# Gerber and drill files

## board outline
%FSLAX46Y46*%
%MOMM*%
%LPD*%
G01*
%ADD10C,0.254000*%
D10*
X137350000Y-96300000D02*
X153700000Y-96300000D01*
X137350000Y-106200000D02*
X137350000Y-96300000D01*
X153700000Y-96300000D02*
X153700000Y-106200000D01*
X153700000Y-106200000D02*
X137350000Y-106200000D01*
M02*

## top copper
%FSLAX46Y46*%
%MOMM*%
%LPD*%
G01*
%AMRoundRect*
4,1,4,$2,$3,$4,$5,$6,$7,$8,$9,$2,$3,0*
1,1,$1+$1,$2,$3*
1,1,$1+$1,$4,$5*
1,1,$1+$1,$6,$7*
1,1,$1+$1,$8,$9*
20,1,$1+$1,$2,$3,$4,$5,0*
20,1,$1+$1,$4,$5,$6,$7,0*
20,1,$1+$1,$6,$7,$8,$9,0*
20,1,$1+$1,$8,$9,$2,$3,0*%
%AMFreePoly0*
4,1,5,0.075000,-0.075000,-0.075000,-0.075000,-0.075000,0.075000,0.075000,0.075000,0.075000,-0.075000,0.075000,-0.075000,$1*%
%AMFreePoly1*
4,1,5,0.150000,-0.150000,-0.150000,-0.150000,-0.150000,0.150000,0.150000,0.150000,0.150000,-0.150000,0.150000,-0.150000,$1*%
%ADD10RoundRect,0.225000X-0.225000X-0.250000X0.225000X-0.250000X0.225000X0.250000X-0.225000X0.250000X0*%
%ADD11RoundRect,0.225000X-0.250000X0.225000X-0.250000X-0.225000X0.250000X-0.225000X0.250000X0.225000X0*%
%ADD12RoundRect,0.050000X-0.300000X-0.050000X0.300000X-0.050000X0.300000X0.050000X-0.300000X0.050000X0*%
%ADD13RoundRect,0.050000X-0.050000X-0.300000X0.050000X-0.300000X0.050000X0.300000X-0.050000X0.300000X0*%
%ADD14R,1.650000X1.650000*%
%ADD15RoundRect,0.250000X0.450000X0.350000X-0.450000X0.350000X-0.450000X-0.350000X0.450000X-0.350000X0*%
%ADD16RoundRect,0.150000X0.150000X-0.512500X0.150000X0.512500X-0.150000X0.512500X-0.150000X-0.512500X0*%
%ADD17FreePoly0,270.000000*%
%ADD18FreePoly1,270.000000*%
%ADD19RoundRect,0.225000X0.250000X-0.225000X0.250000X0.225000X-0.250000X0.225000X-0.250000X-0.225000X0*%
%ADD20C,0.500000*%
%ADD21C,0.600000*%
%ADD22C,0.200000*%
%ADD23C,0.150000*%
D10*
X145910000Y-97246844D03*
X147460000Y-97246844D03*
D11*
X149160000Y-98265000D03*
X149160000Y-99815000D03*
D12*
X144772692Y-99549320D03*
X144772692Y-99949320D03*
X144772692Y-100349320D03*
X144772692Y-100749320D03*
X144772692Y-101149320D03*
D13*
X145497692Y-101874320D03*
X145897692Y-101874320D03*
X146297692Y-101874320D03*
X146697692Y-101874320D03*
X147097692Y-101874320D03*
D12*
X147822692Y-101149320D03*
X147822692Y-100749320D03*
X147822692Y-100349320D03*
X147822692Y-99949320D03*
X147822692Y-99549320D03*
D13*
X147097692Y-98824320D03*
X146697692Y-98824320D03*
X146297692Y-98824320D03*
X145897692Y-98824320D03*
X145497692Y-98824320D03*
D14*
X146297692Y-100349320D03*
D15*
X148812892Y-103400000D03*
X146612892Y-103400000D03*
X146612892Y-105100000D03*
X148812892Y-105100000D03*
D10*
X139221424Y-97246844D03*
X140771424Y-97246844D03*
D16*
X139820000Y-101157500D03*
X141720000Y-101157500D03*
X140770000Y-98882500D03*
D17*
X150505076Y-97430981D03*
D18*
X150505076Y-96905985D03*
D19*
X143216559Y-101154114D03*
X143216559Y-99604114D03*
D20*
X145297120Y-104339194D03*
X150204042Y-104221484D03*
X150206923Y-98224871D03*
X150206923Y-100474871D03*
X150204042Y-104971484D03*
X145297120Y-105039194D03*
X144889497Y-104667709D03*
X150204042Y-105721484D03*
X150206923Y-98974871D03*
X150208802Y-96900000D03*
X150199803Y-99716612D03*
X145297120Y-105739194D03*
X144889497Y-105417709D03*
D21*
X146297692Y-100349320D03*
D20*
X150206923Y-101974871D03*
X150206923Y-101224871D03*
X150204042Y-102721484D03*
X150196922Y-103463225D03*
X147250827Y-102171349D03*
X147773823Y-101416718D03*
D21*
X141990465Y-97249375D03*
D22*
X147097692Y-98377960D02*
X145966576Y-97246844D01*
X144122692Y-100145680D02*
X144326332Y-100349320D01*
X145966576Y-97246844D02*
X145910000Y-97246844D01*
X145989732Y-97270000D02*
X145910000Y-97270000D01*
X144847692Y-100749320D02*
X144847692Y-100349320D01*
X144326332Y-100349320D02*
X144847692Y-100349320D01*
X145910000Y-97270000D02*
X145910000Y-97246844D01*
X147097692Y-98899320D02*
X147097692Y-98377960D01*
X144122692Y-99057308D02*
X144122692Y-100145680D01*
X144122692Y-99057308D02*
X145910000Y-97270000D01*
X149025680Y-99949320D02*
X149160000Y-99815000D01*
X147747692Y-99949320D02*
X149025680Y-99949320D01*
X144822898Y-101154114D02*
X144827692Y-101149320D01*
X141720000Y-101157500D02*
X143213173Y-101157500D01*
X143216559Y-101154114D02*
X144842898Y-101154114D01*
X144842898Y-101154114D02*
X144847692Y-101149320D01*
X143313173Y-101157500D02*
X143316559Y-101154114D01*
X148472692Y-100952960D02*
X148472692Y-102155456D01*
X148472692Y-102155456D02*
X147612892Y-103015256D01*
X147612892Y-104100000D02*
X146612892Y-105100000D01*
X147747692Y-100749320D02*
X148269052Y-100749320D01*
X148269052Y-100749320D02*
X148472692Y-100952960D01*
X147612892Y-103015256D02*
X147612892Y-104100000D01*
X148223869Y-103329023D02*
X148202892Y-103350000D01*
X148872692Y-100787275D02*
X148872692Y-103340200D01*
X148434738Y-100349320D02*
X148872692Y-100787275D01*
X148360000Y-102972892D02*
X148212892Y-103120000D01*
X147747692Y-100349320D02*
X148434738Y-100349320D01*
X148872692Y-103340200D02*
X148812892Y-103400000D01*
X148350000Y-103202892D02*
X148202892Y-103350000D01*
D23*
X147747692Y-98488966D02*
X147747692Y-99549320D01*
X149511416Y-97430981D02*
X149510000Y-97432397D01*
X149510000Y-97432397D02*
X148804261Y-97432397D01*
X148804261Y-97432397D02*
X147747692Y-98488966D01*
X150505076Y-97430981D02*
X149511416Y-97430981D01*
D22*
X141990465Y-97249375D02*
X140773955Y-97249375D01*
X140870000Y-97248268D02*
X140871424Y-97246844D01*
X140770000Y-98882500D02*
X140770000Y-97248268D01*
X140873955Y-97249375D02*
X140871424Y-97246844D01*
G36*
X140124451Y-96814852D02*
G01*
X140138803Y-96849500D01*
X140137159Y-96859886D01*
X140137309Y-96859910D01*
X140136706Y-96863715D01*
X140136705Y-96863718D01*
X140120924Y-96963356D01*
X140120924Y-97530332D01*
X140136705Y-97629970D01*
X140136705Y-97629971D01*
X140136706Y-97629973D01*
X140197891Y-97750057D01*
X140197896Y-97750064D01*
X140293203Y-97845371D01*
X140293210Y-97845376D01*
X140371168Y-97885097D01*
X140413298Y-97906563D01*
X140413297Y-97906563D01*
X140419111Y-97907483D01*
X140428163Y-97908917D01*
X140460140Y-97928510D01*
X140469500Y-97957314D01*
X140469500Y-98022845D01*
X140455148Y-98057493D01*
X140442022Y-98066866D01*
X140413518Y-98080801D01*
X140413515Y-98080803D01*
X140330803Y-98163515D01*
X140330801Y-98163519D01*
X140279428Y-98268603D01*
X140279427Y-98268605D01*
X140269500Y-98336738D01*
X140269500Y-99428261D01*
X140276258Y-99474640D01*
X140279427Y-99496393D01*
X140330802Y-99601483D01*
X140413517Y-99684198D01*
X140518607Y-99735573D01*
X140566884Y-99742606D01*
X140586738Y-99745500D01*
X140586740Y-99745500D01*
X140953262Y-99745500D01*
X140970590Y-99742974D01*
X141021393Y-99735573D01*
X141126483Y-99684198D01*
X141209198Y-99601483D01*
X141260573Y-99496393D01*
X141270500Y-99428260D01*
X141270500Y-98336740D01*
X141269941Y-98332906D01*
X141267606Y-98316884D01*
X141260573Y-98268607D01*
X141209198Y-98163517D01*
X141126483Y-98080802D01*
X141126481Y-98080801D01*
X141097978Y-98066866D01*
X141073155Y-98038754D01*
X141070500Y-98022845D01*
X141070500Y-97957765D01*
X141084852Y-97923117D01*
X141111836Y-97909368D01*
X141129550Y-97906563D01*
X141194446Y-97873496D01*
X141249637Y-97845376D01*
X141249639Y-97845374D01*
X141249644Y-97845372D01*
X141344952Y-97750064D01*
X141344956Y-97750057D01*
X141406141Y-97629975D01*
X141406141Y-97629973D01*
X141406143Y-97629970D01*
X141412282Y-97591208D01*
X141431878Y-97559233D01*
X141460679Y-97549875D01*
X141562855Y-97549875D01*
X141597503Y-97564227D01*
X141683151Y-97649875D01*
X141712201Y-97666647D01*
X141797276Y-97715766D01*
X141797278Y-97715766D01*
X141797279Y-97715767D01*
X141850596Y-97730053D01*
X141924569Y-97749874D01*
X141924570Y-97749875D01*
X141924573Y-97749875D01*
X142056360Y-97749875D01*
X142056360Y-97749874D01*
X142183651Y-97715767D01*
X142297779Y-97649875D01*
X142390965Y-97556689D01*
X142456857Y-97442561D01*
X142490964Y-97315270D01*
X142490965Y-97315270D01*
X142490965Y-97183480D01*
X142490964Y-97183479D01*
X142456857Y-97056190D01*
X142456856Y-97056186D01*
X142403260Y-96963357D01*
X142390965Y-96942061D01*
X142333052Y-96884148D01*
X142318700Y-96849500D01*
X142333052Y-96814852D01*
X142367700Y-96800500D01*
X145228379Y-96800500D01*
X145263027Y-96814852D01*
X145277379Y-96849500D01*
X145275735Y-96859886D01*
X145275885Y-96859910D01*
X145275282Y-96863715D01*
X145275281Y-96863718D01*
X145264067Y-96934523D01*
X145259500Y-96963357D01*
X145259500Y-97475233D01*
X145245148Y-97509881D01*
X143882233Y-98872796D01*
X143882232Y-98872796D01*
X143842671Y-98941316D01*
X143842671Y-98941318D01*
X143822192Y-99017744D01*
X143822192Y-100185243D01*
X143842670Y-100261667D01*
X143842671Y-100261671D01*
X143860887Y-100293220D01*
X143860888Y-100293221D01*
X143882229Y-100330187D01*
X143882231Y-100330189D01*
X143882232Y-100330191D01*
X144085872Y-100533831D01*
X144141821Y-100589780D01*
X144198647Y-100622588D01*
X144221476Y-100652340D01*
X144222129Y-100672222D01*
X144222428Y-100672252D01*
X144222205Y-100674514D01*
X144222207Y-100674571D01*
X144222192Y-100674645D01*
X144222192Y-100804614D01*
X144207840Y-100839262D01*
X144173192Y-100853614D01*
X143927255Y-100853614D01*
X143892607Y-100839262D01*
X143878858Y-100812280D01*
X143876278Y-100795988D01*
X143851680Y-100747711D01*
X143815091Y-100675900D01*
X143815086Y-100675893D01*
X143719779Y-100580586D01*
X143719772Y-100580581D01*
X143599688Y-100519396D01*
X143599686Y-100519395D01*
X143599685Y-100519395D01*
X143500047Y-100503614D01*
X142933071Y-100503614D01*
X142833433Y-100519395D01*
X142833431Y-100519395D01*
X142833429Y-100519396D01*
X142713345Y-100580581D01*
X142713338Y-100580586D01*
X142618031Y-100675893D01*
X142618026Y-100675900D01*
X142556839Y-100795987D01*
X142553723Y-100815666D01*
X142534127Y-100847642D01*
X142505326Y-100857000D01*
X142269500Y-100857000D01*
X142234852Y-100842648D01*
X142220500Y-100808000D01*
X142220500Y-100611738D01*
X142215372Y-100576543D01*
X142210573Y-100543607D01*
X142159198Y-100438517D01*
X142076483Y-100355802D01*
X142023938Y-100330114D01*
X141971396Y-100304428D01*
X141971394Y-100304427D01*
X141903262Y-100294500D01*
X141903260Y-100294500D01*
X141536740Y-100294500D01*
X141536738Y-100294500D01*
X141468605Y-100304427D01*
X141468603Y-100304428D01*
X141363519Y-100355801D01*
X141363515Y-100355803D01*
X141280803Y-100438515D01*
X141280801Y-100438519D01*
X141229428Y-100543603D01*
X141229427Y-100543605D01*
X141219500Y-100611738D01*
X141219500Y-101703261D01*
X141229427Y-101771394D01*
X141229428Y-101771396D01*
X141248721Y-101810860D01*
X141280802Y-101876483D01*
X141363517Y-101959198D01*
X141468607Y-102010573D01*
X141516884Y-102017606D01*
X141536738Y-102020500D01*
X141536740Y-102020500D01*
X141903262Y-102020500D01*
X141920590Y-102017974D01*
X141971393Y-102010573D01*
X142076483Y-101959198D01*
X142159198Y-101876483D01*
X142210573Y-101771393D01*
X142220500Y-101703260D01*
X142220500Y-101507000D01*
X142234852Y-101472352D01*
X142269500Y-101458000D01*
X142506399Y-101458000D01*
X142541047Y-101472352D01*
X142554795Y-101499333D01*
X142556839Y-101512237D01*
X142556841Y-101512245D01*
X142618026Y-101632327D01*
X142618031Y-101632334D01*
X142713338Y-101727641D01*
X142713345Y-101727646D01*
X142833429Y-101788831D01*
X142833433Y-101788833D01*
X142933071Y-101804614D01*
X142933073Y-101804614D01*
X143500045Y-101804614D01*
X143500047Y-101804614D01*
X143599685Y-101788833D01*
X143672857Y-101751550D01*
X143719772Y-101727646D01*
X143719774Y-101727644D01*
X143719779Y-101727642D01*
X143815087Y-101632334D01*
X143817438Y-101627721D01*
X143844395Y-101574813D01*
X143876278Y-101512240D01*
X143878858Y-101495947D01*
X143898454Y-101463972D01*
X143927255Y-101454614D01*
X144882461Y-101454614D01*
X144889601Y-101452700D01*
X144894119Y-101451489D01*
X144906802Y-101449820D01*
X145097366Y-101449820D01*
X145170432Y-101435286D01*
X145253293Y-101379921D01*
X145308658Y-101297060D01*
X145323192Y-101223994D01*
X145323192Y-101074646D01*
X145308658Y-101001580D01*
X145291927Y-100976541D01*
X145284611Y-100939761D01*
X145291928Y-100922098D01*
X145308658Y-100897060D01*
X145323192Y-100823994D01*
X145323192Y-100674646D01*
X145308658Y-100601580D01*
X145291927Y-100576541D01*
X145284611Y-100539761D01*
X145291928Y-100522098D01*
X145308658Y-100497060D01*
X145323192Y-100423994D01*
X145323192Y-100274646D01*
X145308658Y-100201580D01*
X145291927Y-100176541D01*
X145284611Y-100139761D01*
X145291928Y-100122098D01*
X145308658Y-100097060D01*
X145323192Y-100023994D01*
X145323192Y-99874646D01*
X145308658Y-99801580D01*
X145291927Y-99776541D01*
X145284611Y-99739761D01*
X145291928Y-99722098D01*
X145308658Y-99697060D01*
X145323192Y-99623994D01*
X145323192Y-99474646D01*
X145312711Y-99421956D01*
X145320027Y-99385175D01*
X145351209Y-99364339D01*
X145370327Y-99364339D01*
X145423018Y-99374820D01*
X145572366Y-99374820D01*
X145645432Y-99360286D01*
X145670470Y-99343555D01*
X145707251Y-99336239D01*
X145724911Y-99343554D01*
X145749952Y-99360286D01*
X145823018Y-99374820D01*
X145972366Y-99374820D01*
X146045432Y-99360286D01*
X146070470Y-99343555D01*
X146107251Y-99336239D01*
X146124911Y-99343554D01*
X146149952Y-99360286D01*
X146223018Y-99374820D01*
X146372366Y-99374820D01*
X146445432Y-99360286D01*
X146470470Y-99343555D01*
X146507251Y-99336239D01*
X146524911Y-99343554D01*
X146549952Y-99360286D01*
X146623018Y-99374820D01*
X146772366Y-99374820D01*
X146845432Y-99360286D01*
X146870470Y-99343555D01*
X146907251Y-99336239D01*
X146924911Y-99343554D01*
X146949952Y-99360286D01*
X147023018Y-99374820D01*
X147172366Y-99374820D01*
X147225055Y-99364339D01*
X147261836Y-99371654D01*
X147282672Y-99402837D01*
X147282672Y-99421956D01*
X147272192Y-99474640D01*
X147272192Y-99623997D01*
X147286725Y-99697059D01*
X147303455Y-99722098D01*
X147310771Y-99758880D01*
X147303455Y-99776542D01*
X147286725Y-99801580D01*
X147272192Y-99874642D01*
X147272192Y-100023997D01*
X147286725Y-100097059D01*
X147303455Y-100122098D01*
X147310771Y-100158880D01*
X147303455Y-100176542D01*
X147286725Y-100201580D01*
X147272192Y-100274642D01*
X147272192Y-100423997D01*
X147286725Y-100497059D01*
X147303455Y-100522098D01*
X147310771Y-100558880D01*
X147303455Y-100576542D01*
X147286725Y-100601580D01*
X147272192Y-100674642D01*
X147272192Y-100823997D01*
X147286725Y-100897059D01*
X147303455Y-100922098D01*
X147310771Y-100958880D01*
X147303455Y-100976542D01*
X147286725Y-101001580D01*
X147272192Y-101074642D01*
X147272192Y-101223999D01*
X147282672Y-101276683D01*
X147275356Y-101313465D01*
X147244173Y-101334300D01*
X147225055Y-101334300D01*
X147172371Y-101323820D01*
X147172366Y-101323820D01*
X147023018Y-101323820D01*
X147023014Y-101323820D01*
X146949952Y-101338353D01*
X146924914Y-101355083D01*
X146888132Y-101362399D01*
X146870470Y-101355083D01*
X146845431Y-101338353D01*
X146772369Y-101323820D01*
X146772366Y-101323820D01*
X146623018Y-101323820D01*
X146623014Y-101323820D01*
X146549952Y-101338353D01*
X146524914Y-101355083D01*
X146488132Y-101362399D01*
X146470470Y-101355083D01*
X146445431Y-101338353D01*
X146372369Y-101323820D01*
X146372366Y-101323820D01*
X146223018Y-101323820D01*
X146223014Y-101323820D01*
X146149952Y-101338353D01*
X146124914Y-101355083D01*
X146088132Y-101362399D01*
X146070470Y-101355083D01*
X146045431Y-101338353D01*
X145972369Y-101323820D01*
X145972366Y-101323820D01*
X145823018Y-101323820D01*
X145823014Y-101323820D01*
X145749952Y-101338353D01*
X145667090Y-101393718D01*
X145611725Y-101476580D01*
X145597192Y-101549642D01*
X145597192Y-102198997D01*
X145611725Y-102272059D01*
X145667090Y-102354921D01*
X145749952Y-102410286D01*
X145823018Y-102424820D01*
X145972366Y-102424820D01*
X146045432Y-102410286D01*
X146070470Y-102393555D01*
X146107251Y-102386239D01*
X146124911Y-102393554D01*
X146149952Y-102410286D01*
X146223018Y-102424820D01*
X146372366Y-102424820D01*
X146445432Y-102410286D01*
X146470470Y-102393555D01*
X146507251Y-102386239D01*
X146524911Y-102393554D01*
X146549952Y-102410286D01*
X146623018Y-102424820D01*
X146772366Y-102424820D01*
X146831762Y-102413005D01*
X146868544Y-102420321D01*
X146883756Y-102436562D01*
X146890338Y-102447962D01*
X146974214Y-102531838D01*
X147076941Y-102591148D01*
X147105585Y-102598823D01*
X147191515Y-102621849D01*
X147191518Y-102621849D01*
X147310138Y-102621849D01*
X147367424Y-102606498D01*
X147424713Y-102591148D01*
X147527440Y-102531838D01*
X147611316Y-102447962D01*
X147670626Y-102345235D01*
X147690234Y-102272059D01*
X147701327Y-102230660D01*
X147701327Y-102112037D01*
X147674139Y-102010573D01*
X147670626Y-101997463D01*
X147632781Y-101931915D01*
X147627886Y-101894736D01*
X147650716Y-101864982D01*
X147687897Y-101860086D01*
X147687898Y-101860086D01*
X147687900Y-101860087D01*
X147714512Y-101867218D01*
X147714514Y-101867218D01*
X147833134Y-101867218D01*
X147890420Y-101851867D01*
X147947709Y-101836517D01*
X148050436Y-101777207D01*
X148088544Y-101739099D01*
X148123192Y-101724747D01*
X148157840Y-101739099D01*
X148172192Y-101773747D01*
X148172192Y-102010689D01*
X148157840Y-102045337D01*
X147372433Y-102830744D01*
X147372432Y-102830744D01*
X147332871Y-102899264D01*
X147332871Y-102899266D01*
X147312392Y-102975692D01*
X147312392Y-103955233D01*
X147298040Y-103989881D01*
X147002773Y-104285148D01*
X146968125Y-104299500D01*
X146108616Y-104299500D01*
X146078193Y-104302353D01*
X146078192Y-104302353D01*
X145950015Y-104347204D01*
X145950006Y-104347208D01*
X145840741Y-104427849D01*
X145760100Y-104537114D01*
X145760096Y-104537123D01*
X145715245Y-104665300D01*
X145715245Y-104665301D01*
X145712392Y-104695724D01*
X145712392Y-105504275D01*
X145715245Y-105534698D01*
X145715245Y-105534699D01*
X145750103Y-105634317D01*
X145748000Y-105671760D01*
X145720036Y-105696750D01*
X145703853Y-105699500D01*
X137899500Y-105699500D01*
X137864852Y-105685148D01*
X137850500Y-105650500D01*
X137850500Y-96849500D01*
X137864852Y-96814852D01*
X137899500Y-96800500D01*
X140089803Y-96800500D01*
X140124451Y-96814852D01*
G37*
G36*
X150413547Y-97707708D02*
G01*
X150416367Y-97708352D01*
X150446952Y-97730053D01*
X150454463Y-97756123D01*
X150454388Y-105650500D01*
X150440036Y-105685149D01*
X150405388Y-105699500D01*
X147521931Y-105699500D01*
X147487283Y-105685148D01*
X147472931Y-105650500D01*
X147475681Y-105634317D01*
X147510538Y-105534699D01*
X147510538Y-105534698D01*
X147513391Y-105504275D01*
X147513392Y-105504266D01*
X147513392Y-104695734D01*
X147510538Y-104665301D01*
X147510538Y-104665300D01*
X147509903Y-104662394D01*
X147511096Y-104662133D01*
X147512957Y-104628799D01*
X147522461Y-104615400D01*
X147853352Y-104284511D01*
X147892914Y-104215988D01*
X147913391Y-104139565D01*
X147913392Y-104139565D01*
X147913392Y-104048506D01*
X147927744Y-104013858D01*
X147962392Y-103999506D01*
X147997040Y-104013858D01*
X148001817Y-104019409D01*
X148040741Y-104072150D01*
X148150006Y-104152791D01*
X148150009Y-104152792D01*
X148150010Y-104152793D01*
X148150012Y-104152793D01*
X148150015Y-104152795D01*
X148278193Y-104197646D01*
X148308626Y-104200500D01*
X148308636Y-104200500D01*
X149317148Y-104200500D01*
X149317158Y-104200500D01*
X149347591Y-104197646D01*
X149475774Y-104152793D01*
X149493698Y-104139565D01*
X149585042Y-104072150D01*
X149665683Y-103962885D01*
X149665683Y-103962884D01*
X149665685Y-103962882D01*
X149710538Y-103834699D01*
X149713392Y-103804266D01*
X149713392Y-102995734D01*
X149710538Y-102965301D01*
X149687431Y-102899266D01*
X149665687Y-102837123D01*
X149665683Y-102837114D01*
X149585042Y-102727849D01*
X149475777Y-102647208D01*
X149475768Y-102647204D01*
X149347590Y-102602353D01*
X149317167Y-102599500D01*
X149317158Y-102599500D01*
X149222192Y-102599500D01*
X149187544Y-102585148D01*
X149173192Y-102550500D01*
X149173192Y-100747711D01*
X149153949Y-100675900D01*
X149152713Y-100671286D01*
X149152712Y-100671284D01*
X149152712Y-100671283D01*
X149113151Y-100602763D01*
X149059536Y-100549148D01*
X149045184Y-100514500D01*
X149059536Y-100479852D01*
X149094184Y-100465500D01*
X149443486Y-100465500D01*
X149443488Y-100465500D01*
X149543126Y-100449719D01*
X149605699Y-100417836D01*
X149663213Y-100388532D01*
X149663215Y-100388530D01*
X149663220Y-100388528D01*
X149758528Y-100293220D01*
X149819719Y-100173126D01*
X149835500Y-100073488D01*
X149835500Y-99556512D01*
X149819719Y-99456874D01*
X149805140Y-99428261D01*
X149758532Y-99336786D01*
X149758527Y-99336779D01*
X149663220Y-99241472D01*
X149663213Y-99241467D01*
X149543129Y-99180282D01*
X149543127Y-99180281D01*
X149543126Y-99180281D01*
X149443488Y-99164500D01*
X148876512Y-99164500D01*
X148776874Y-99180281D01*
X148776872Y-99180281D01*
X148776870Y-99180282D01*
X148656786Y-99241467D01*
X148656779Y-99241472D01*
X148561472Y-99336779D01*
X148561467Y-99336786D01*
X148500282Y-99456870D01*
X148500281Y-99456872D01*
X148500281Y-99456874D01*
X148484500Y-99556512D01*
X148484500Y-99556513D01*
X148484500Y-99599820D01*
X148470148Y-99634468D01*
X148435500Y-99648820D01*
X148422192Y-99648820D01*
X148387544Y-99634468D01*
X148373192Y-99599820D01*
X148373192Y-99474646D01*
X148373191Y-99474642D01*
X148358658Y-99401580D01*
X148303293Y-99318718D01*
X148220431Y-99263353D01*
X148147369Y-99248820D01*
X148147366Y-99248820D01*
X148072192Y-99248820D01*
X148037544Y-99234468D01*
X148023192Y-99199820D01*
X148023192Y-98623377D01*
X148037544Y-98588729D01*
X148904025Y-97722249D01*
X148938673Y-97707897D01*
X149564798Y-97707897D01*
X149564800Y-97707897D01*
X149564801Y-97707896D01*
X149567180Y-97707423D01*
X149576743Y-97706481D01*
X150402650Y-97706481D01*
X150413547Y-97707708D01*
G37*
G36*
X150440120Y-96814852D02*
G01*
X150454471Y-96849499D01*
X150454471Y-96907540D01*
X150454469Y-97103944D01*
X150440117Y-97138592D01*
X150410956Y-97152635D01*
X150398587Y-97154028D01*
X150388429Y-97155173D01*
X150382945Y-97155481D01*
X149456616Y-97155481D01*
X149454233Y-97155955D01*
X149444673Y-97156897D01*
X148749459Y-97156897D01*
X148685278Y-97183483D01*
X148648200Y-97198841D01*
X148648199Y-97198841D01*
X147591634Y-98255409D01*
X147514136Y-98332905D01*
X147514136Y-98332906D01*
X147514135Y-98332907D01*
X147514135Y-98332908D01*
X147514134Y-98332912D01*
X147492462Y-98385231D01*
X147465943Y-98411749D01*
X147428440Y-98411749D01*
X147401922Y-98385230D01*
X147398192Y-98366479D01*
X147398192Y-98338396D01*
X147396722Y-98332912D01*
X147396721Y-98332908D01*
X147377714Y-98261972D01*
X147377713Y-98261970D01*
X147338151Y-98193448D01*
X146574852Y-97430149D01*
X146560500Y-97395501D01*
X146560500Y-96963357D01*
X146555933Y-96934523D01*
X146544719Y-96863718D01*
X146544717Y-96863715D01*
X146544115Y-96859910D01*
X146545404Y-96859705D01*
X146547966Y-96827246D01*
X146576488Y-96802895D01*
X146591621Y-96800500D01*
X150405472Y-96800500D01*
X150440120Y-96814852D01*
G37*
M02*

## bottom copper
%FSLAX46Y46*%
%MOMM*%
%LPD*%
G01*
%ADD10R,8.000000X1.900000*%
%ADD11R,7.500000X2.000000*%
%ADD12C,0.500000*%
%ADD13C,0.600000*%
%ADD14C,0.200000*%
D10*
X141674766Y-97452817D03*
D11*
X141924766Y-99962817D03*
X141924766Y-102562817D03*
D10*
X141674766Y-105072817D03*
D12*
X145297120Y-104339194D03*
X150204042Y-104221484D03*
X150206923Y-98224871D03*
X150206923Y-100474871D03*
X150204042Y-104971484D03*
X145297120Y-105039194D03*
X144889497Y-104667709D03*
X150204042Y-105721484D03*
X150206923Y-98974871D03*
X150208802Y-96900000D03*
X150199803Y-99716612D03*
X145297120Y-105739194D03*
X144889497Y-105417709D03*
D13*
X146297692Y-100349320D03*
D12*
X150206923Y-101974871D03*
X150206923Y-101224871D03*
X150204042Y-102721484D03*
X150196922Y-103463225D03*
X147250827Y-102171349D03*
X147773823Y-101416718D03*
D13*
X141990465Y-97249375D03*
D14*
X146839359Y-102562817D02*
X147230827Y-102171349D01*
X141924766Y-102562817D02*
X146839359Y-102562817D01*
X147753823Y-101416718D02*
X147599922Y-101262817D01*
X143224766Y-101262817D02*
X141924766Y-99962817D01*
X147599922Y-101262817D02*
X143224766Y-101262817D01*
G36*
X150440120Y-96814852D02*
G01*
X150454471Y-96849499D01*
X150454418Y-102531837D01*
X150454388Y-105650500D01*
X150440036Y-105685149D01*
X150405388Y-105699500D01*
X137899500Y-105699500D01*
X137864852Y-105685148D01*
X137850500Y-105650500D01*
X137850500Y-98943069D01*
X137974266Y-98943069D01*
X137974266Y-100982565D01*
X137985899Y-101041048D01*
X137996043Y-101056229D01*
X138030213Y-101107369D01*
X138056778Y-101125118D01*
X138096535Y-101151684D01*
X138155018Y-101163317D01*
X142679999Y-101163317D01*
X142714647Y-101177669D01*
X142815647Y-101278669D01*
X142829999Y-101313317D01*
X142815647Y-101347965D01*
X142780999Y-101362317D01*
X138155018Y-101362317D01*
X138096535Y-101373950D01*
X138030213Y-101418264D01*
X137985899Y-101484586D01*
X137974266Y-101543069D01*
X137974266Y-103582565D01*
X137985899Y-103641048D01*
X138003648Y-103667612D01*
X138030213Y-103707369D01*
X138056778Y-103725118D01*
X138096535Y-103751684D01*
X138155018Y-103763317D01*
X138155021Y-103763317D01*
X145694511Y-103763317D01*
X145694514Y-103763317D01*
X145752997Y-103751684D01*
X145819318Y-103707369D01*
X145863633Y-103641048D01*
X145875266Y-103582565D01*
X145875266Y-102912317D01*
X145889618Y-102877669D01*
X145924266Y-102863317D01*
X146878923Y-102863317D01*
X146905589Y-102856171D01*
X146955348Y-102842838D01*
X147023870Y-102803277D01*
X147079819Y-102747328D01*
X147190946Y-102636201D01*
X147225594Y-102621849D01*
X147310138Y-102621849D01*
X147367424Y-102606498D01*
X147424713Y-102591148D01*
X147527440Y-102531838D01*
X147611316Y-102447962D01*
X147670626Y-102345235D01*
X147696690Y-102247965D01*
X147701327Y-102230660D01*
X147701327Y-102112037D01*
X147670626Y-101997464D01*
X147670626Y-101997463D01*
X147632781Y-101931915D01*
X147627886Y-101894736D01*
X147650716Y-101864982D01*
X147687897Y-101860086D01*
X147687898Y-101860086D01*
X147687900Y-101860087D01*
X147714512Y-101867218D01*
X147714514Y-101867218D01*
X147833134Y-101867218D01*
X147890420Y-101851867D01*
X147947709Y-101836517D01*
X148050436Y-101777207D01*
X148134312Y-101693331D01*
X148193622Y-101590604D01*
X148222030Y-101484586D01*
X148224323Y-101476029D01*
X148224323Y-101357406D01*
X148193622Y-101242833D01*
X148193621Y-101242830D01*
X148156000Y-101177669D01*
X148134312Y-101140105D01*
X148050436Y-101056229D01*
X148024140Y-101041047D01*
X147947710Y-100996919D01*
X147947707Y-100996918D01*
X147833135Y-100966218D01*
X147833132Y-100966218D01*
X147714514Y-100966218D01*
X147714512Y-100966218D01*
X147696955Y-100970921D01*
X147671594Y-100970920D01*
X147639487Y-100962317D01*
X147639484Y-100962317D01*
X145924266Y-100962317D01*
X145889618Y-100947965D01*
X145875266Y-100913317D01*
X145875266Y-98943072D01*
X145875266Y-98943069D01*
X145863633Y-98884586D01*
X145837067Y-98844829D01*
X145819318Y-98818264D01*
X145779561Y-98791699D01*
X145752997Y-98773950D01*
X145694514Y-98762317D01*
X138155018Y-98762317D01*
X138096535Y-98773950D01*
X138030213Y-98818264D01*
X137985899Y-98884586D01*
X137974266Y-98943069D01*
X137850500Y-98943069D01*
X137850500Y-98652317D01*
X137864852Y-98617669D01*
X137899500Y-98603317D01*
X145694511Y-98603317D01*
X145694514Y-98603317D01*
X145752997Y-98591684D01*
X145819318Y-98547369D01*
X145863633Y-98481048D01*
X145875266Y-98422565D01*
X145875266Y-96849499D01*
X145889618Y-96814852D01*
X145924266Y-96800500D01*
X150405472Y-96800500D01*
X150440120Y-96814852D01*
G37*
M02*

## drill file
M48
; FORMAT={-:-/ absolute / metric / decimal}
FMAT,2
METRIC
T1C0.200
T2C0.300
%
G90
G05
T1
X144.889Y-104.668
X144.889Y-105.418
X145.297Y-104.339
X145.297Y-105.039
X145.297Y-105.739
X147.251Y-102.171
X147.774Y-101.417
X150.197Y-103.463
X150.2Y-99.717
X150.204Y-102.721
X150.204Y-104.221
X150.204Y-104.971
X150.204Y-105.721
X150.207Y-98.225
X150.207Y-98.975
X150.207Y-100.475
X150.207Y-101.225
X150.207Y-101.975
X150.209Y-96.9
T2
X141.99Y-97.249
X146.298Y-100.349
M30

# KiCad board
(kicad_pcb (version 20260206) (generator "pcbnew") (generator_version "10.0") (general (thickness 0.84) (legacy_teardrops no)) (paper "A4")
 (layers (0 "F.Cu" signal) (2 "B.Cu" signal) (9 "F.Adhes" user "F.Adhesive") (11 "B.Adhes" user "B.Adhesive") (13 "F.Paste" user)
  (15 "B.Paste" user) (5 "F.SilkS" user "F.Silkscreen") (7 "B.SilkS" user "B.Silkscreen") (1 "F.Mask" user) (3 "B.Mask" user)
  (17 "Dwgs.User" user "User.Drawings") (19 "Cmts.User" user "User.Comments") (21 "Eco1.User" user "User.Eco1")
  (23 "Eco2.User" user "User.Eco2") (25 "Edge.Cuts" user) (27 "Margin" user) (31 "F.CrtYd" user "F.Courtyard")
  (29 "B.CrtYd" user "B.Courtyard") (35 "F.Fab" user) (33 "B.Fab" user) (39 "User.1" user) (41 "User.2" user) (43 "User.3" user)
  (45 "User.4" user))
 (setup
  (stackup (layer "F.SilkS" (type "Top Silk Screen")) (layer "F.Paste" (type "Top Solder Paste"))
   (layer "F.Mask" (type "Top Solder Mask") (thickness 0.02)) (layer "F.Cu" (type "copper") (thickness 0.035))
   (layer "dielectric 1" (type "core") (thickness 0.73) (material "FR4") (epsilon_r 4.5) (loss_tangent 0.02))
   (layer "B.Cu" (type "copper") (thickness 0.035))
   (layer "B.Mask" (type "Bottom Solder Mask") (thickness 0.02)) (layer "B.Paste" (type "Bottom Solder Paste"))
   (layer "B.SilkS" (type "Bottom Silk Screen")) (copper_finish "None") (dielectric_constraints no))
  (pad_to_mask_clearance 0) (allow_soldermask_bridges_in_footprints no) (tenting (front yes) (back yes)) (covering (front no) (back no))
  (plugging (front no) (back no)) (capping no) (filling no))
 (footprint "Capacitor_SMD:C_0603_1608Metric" (layer "F.Cu") (at 146.685 97.246844)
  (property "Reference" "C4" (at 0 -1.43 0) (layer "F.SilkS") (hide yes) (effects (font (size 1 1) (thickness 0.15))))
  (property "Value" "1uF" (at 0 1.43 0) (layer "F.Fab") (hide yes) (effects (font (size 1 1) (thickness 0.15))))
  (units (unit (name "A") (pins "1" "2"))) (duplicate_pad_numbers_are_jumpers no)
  (pad "1" smd roundrect (at -0.775 0) (size 0.9 0.95) (layers "F.Cu" "F.Mask" "F.Paste") (roundrect_rratio 0.25) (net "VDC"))
  (pad "2" smd roundrect (at 0.775 0) (size 0.9 0.95) (layers "F.Cu" "F.Mask" "F.Paste") (roundrect_rratio 0.25) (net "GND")))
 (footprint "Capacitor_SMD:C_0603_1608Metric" (layer "F.Cu") (at 149.16 99.04 -90)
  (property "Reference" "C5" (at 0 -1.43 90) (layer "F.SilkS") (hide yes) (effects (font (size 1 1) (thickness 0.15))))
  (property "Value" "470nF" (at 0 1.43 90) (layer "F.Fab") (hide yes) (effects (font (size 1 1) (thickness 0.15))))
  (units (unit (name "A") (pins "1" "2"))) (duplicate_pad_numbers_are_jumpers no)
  (pad "1" smd roundrect (at -0.775 0 270) (size 0.9 0.95) (layers "F.Cu" "F.Mask" "F.Paste") (roundrect_rratio 0.25) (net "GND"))
  (pad "2" smd roundrect (at 0.775 0 270) (size 0.9 0.95) (layers "F.Cu" "F.Mask" "F.Paste") (roundrect_rratio 0.25) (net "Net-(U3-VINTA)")))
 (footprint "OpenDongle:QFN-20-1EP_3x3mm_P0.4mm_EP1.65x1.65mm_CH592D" (layer "F.Cu") (at 146.297692 100.34932)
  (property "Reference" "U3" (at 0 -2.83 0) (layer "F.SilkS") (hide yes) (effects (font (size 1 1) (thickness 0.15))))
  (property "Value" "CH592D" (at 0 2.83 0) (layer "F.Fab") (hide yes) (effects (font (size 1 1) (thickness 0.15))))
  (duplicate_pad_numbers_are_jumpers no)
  (pad "" smd roundrect (at -0.41 -0.41) (size 0.67 0.67) (layers "F.Paste") (roundrect_rratio 0.25))
  (pad "" smd roundrect (at -0.41 0.41) (size 0.67 0.67) (layers "F.Paste") (roundrect_rratio 0.25))
  (pad "" smd roundrect (at 0.41 -0.41) (size 0.67 0.67) (layers "F.Paste") (roundrect_rratio 0.25))
  (pad "" smd roundrect (at 0.41 0.41) (size 0.67 0.67) (layers "F.Paste") (roundrect_rratio 0.25))
  (pad "1" smd roundrect (at -1.525 -0.8) (size 0.7 0.2) (layers "F.Cu" "F.Mask" "F.Paste") (roundrect_rratio 0.25)
   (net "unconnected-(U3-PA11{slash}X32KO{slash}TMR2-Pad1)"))
  (pad "2" smd roundrect (at -1.525 -0.4) (size 0.7 0.2) (layers "F.Cu" "F.Mask" "F.Paste") (roundrect_rratio 0.25)
   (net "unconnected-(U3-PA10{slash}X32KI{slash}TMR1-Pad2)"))
  (pad "3" smd roundrect (at -1.525 0) (size 0.7 0.2) (layers "F.Cu" "F.Mask" "F.Paste") (roundrect_rratio 0.25) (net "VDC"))
  (pad "4" smd roundrect (at -1.525 0.4) (size 0.7 0.2) (layers "F.Cu" "F.Mask" "F.Paste") (roundrect_rratio 0.25) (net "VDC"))
  (pad "5" smd roundrect (at -1.525 0.8) (size 0.7 0.2) (layers "F.Cu" "F.Mask" "F.Paste") (roundrect_rratio 0.25) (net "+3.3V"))
  (pad "6" smd roundrect (at -0.8 1.525) (size 0.2 0.7) (layers "F.Cu" "F.Mask" "F.Paste") (roundrect_rratio 0.25) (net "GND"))
  (pad "7" smd roundrect (at -0.4 1.525) (size 0.2 0.7) (layers "F.Cu" "F.Mask" "F.Paste") (roundrect_rratio 0.25)
   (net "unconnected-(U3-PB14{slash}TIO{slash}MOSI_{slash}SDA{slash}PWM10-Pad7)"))
  (pad "8" smd roundrect (at 0 1.525) (size 0.2 0.7) (layers "F.Cu" "F.Mask" "F.Paste") (roundrect_rratio 0.25)
   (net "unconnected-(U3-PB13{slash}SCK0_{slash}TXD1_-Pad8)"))
  (pad "9" smd roundrect (at 0.4 1.525) (size 0.2 0.7) (layers "F.Cu" "F.Mask" "F.Paste") (roundrect_rratio 0.25)
   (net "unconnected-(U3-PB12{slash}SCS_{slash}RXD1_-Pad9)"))
  (pad "10" smd roundrect (at 0.8 1.525) (size 0.2 0.7) (layers "F.Cu" "F.Mask" "F.Paste") (roundrect_rratio 0.25) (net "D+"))
  (pad "11" smd roundrect (at 1.525 0.8) (size 0.7 0.2) (layers "F.Cu" "F.Mask" "F.Paste") (roundrect_rratio 0.25) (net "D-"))
  (pad "12" smd roundrect (at 1.525 0.4) (size 0.7 0.2) (layers "F.Cu" "F.Mask" "F.Paste") (roundrect_rratio 0.25) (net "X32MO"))
  (pad "13" smd roundrect (at 1.525 0) (size 0.7 0.2) (layers "F.Cu" "F.Mask" "F.Paste") (roundrect_rratio 0.25) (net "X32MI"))
  (pad "14" smd roundrect (at 1.525 -0.4) (size 0.7 0.2) (layers "F.Cu" "F.Mask" "F.Paste") (roundrect_rratio 0.25) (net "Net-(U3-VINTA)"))
  (pad "15" smd roundrect (at 1.525 -0.8) (size 0.7 0.2) (layers "F.Cu" "F.Mask" "F.Paste") (roundrect_rratio 0.25) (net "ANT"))
  (pad "16" smd roundrect (at 0.8 -1.525) (size 0.2 0.7) (layers "F.Cu" "F.Mask" "F.Paste") (roundrect_rratio 0.25) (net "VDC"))
  (pad "17" smd roundrect (at 0.4 -1.525) (size 0.2 0.7) (layers "F.Cu" "F.Mask" "F.Paste") (roundrect_rratio 0.25)
   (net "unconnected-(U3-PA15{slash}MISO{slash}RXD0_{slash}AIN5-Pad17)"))
  (pad "18" smd roundrect (at 0 -1.525) (size 0.2 0.7) (layers "F.Cu" "F.Mask" "F.Paste") (roundrect_rratio 0.25)
   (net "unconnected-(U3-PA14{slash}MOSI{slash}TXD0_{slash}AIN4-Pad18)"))
  (pad "19" smd roundrect (at -0.4 -1.525) (size 0.2 0.7) (layers "F.Cu" "F.Mask" "F.Paste") (roundrect_rratio 0.25)
   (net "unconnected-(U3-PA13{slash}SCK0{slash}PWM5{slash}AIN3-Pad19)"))
  (pad "20" smd roundrect (at -0.8 -1.525) (size 0.2 0.7) (layers "F.Cu" "F.Mask" "F.Paste") (roundrect_rratio 0.25)
   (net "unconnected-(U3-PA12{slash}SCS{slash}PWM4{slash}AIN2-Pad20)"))
  (pad "21" smd rect (at 0 0) (size 1.65 1.65) (layers "F.Cu" "F.Mask") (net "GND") (zone_connect 2)))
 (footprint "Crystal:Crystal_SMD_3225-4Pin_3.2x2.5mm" (layer "F.Cu") (at 147.712892 104.25 180)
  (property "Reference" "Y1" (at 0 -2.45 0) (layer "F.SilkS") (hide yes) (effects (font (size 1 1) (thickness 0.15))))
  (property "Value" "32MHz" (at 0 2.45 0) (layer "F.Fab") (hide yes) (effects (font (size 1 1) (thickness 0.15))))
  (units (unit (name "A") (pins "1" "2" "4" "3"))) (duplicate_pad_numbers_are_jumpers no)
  (pad "1" smd roundrect (at -1.1 0.85 180) (size 1.4 1.2) (layers "F.Cu" "F.Mask" "F.Paste") (roundrect_rratio 0.208333) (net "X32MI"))
  (pad "2" smd roundrect (at 1.1 0.85 180) (size 1.4 1.2) (layers "F.Cu" "F.Mask" "F.Paste") (roundrect_rratio 0.208333) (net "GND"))
  (pad "3" smd roundrect (at 1.1 -0.85 180) (size 1.4 1.2) (layers "F.Cu" "F.Mask" "F.Paste") (roundrect_rratio 0.208333) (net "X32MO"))
  (pad "4" smd roundrect (at -1.1 -0.85 180) (size 1.4 1.2) (layers "F.Cu" "F.Mask" "F.Paste") (roundrect_rratio 0.208333) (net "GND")))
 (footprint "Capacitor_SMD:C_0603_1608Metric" (layer "F.Cu") (at 139.996424 97.246844)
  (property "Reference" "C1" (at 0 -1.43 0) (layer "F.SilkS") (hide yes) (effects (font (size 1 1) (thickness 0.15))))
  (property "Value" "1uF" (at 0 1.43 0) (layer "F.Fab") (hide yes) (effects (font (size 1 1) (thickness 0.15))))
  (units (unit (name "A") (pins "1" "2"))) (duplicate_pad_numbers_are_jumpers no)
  (pad "1" smd roundrect (at -0.775 0) (size 0.9 0.95) (layers "F.Cu" "F.Mask" "F.Paste") (roundrect_rratio 0.25) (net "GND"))
  (pad "2" smd roundrect (at 0.775 0) (size 0.9 0.95) (layers "F.Cu" "F.Mask" "F.Paste") (roundrect_rratio 0.25) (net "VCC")))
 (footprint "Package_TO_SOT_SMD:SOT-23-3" (layer "F.Cu") (at 140.77 100.02 90)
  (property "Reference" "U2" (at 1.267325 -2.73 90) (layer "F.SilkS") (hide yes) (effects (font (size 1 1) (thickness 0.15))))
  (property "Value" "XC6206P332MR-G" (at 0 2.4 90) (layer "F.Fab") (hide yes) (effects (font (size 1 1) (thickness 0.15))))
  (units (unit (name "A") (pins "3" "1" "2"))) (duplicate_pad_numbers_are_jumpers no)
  (pad "1" smd roundrect (at -1.1375 -0.95 90) (size 1.325 0.6) (layers "F.Cu" "F.Mask" "F.Paste") (roundrect_rratio 0.25) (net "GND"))
  (pad "2" smd roundrect (at -1.1375 0.95 90) (size 1.325 0.6) (layers "F.Cu" "F.Mask" "F.Paste") (roundrect_rratio 0.25) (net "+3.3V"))
  (pad "3" smd roundrect (at 1.1375 0 90) (size 1.325 0.6) (layers "F.Cu" "F.Mask" "F.Paste") (roundrect_rratio 0.25) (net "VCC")))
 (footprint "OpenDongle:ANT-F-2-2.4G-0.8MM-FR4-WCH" (layer "F.Cu") (at 151.800076 101.240981 -90)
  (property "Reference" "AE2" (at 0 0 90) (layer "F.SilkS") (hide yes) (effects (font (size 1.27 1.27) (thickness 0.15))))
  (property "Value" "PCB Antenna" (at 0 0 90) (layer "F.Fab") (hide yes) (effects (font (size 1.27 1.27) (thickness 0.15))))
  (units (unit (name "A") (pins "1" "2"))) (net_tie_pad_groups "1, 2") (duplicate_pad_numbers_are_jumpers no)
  (pad "1" smd custom (at -3.81 1.295 270) (size 0.15 0.15) (layers "F.Cu") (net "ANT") (solder_mask_margin 0.1016)
   (options (clearance outline) (anchor rect)) (primitives)
   (teardrops (best_length_ratio 0.5) (max_length 1) (best_width_ratio 1) (max_width 2) (curved_edges no) (filter_ratio 0.9) (enabled yes)
    (allow_two_segments yes) (prefer_zone_connections yes)))
  (pad "2" smd custom (at -4.334996 1.295 270) (size 0.3 0.3) (layers "F.Cu") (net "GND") (solder_mask_margin 0.1016)
   (options (clearance outline) (anchor rect)) (primitives)))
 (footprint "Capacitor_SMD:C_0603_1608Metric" (layer "F.Cu") (at 143.216559 100.379114 90)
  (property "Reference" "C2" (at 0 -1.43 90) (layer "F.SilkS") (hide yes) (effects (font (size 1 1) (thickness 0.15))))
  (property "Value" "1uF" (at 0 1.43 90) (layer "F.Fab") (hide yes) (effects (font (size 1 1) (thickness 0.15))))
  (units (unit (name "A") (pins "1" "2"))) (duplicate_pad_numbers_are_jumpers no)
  (pad "1" smd roundrect (at -0.775 0 90) (size 0.9 0.95) (layers "F.Cu" "F.Mask" "F.Paste") (roundrect_rratio 0.25) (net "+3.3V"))
  (pad "2" smd roundrect (at 0.775 0 90) (size 0.9 0.95) (layers "F.Cu" "F.Mask" "F.Paste") (roundrect_rratio 0.25) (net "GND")))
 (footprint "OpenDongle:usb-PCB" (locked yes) (layer "B.Cu") (at 136.774766 101.262817 90)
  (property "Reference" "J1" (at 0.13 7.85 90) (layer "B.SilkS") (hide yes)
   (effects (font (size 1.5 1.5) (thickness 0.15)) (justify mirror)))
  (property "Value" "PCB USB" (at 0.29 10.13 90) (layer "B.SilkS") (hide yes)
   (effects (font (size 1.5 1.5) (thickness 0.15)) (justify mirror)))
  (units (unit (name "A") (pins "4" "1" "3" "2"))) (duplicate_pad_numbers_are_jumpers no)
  (pad "1" connect rect (at 3.81 4.9 90) (size 1.9 8) (layers "B.Cu" "B.Mask") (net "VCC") (thermal_bridge_angle 45))
  (pad "2" connect rect (at 1.3 5.15 90) (size 2 7.5) (layers "B.Cu" "B.Mask") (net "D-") (thermal_bridge_angle 45))
  (pad "3" connect rect (at -1.3 5.15 90) (size 2 7.5) (layers "B.Cu" "B.Mask") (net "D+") (thermal_bridge_angle 45))
  (pad "4" connect rect (at -3.81 4.9 90) (size 1.9 8) (layers "B.Cu" "B.Mask") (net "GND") (thermal_bridge_angle 45)))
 (gr_line (start 137.35 96.3) (end 153.7 96.3) (stroke (width 0.254) (type default)) (layer "Edge.Cuts"))
 (gr_line (start 137.35 106.2) (end 137.35 96.3) (stroke (width 0.254) (type default)) (layer "Edge.Cuts"))
 (gr_line (start 153.7 96.3) (end 153.7 106.2) (stroke (width 0.254) (type default)) (layer "Edge.Cuts"))
 (gr_line (start 153.7 106.2) (end 137.35 106.2) (stroke (width 0.254) (type default)) (layer "Edge.Cuts"))
 (segment (start 147.097692 98.37796) (end 145.966576 97.246844) (width 0.2) (layer "F.Cu") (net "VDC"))
 (segment (start 144.122692 100.14568) (end 144.326332 100.34932) (width 0.2) (layer "F.Cu") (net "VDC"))
 (segment (start 145.966576 97.246844) (end 145.91 97.246844) (width 0.2) (layer "F.Cu") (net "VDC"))
 (segment (start 145.989732 97.27) (end 145.91 97.27) (width 0.2) (layer "F.Cu") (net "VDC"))
 (segment (start 144.847692 100.74932) (end 144.847692 100.34932) (width 0.2) (layer "F.Cu") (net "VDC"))
 (segment (start 144.326332 100.34932) (end 144.847692 100.34932) (width 0.2) (layer "F.Cu") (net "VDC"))
 (segment (start 145.91 97.27) (end 145.91 97.246844) (width 0.2) (layer "F.Cu") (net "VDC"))
 (segment (start 147.097692 98.89932) (end 147.097692 98.37796) (width 0.2) (layer "F.Cu") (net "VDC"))
 (segment (start 144.122692 99.057308) (end 144.122692 100.14568) (width 0.2) (layer "F.Cu") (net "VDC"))
 (segment (start 144.122692 99.057308) (end 145.91 97.27) (width 0.2) (layer "F.Cu") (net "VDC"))
 (via (at 145.29712 104.339194) (size 0.5) (drill 0.2) (layers "F.Cu" "B.Cu") (free yes) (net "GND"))
 (via (at 150.204042 104.221484) (size 0.5) (drill 0.2) (layers "F.Cu" "B.Cu") (free yes) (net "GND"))
 (via (at 150.206923 98.224871) (size 0.5) (drill 0.2) (layers "F.Cu" "B.Cu") (free yes) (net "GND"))
 (via (at 150.206923 100.474871) (size 0.5) (drill 0.2) (layers "F.Cu" "B.Cu") (free yes) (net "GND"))
 (via (at 150.204042 104.971484) (size 0.5) (drill 0.2) (layers "F.Cu" "B.Cu") (free yes) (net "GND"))
 (via (at 145.29712 105.039194) (size 0.5) (drill 0.2) (layers "F.Cu" "B.Cu") (free yes) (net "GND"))
 (via (at 144.889497 104.667709) (size 0.5) (drill 0.2) (layers "F.Cu" "B.Cu") (free yes) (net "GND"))
 (via (at 150.204042 105.721484) (size 0.5) (drill 0.2) (layers "F.Cu" "B.Cu") (free yes) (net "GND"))
 (via (at 150.206923 98.974871) (size 0.5) (drill 0.2) (layers "F.Cu" "B.Cu") (free yes) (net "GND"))
 (via (at 150.208802 96.9) (size 0.5) (drill 0.2) (layers "F.Cu" "B.Cu") (free yes) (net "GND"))
 (via (at 150.199803 99.716612) (size 0.5) (drill 0.2) (layers "F.Cu" "B.Cu") (free yes) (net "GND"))
 (via (at 145.29712 105.739194) (size 0.5) (drill 0.2) (layers "F.Cu" "B.Cu") (free yes) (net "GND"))
 (via (at 144.889497 105.417709) (size 0.5) (drill 0.2) (layers "F.Cu" "B.Cu") (free yes) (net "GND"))
 (via (at 146.297692 100.34932) (size 0.6) (drill 0.3) (layers "F.Cu" "B.Cu") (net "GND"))
 (via (at 150.206923 101.974871) (size 0.5) (drill 0.2) (layers "F.Cu" "B.Cu") (free yes) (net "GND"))
 (via (at 150.206923 101.224871) (size 0.5) (drill 0.2) (layers "F.Cu" "B.Cu") (free yes) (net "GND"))
 (via (at 150.204042 102.721484) (size 0.5) (drill 0.2) (layers "F.Cu" "B.Cu") (free yes) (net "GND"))
 (via (at 150.196922 103.463225) (size 0.5) (drill 0.2) (layers "F.Cu" "B.Cu") (free yes) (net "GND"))
 (segment (start 149.02568 99.94932) (end 149.16 99.815) (width 0.2) (layer "F.Cu") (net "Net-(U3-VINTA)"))
 (segment (start 147.747692 99.94932) (end 149.02568 99.94932) (width 0.2) (layer "F.Cu") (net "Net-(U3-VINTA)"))
 (segment (start 144.822898 101.154114) (end 144.827692 101.14932) (width 0.2) (layer "F.Cu") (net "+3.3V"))
 (segment (start 141.72 101.1575) (end 143.213173 101.1575) (width 0.2) (layer "F.Cu") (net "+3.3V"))
 (segment (start 143.216559 101.154114) (end 144.842898 101.154114) (width 0.2) (layer "F.Cu") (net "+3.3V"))
 (segment (start 144.842898 101.154114) (end 144.847692 101.14932) (width 0.2) (layer "F.Cu") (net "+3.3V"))
 (segment (start 143.313173 101.1575) (end 143.316559 101.154114) (width 0.2) (layer "F.Cu") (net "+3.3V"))
 (via (at 147.250827 102.171349) (size 0.5) (drill 0.2) (layers "F.Cu" "B.Cu") (free yes) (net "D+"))
 (segment (start 146.839359 102.562817) (end 147.230827 102.171349) (width 0.2) (layer "B.Cu") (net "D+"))
 (segment (start 141.924766 102.562817) (end 146.839359 102.562817) (width 0.2) (layer "B.Cu") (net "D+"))
 (via (at 147.773823 101.416718) (size 0.5) (drill 0.2) (layers "F.Cu" "B.Cu") (free yes) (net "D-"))
 (segment (start 147.753823 101.416718) (end 147.599922 101.262817) (width 0.2) (layer "B.Cu") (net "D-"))
 (segment (start 143.224766 101.262817) (end 141.924766 99.962817) (width 0.2) (layer "B.Cu") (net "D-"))
 (segment (start 147.599922 101.262817) (end 143.224766 101.262817) (width 0.2) (layer "B.Cu") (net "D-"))
 (segment (start 148.472692 100.95296) (end 148.472692 102.155456) (width 0.2) (layer "F.Cu") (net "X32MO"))
 (segment (start 148.472692 102.155456) (end 147.612892 103.015256) (width 0.2) (layer "F.Cu") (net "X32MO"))
 (segment (start 147.612892 104.1) (end 146.612892 105.1) (width 0.2) (layer "F.Cu") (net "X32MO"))
 (segment (start 147.747692 100.74932) (end 148.269052 100.74932) (width 0.2) (layer "F.Cu") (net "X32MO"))
 (segment (start 148.269052 100.74932) (end 148.472692 100.95296) (width 0.2) (layer "F.Cu") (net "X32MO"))
 (segment (start 147.612892 103.015256) (end 147.612892 104.1) (width 0.2) (layer "F.Cu") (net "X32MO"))
 (segment (start 148.223869 103.329023) (end 148.202892 103.35) (width 0.2) (layer "F.Cu") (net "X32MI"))
 (segment (start 148.872692 100.787275) (end 148.872692 103.3402) (width 0.2) (layer "F.Cu") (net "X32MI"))
 (segment (start 148.434738 100.34932) (end 148.872692 100.787275) (width 0.2) (layer "F.Cu") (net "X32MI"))
 (segment (start 148.36 102.972892) (end 148.212892 103.12) (width 0.2) (layer "F.Cu") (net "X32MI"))
 (segment (start 147.747692 100.34932) (end 148.434738 100.34932) (width 0.2) (layer "F.Cu") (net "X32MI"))
 (segment (start 148.872692 103.3402) (end 148.812892 103.4) (width 0.2) (layer "F.Cu") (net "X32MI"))
 (segment (start 148.35 103.202892) (end 148.202892 103.35) (width 0.2) (layer "F.Cu") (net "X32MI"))
 (segment (start 147.747692 98.488966) (end 147.747692 99.54932) (width 0.15) (layer "F.Cu") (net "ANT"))
 (segment (start 149.511416 97.430981) (end 149.51 97.432397) (width 0.15) (layer "F.Cu") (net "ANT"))
 (segment (start 149.51 97.432397) (end 148.804261 97.432397) (width 0.15) (layer "F.Cu") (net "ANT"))
 (segment (start 148.804261 97.432397) (end 147.747692 98.488966) (width 0.15) (layer "F.Cu") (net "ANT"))
 (segment (start 150.505076 97.430981) (end 149.511416 97.430981) (width 0.15) (layer "F.Cu") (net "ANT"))
 (segment (start 141.990465 97.249375) (end 140.773955 97.249375) (width 0.2) (layer "F.Cu") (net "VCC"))
 (segment (start 140.87 97.248268) (end 140.871424 97.246844) (width 0.2) (layer "F.Cu") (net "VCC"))
 (segment (start 140.77 98.8825) (end 140.77 97.248268) (width 0.2) (layer "F.Cu") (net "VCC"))
 (segment (start 140.873955 97.249375) (end 140.871424 97.246844) (width 0.2) (layer "F.Cu") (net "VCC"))
 (via (at 141.990465 97.249375) (size 0.6) (drill 0.3) (layers "F.Cu" "B.Cu") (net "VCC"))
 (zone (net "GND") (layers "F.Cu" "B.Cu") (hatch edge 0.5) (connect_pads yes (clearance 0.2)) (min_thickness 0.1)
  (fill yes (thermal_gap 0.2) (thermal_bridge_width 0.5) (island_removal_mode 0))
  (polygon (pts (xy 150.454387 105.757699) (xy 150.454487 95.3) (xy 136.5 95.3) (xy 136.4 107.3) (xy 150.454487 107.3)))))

